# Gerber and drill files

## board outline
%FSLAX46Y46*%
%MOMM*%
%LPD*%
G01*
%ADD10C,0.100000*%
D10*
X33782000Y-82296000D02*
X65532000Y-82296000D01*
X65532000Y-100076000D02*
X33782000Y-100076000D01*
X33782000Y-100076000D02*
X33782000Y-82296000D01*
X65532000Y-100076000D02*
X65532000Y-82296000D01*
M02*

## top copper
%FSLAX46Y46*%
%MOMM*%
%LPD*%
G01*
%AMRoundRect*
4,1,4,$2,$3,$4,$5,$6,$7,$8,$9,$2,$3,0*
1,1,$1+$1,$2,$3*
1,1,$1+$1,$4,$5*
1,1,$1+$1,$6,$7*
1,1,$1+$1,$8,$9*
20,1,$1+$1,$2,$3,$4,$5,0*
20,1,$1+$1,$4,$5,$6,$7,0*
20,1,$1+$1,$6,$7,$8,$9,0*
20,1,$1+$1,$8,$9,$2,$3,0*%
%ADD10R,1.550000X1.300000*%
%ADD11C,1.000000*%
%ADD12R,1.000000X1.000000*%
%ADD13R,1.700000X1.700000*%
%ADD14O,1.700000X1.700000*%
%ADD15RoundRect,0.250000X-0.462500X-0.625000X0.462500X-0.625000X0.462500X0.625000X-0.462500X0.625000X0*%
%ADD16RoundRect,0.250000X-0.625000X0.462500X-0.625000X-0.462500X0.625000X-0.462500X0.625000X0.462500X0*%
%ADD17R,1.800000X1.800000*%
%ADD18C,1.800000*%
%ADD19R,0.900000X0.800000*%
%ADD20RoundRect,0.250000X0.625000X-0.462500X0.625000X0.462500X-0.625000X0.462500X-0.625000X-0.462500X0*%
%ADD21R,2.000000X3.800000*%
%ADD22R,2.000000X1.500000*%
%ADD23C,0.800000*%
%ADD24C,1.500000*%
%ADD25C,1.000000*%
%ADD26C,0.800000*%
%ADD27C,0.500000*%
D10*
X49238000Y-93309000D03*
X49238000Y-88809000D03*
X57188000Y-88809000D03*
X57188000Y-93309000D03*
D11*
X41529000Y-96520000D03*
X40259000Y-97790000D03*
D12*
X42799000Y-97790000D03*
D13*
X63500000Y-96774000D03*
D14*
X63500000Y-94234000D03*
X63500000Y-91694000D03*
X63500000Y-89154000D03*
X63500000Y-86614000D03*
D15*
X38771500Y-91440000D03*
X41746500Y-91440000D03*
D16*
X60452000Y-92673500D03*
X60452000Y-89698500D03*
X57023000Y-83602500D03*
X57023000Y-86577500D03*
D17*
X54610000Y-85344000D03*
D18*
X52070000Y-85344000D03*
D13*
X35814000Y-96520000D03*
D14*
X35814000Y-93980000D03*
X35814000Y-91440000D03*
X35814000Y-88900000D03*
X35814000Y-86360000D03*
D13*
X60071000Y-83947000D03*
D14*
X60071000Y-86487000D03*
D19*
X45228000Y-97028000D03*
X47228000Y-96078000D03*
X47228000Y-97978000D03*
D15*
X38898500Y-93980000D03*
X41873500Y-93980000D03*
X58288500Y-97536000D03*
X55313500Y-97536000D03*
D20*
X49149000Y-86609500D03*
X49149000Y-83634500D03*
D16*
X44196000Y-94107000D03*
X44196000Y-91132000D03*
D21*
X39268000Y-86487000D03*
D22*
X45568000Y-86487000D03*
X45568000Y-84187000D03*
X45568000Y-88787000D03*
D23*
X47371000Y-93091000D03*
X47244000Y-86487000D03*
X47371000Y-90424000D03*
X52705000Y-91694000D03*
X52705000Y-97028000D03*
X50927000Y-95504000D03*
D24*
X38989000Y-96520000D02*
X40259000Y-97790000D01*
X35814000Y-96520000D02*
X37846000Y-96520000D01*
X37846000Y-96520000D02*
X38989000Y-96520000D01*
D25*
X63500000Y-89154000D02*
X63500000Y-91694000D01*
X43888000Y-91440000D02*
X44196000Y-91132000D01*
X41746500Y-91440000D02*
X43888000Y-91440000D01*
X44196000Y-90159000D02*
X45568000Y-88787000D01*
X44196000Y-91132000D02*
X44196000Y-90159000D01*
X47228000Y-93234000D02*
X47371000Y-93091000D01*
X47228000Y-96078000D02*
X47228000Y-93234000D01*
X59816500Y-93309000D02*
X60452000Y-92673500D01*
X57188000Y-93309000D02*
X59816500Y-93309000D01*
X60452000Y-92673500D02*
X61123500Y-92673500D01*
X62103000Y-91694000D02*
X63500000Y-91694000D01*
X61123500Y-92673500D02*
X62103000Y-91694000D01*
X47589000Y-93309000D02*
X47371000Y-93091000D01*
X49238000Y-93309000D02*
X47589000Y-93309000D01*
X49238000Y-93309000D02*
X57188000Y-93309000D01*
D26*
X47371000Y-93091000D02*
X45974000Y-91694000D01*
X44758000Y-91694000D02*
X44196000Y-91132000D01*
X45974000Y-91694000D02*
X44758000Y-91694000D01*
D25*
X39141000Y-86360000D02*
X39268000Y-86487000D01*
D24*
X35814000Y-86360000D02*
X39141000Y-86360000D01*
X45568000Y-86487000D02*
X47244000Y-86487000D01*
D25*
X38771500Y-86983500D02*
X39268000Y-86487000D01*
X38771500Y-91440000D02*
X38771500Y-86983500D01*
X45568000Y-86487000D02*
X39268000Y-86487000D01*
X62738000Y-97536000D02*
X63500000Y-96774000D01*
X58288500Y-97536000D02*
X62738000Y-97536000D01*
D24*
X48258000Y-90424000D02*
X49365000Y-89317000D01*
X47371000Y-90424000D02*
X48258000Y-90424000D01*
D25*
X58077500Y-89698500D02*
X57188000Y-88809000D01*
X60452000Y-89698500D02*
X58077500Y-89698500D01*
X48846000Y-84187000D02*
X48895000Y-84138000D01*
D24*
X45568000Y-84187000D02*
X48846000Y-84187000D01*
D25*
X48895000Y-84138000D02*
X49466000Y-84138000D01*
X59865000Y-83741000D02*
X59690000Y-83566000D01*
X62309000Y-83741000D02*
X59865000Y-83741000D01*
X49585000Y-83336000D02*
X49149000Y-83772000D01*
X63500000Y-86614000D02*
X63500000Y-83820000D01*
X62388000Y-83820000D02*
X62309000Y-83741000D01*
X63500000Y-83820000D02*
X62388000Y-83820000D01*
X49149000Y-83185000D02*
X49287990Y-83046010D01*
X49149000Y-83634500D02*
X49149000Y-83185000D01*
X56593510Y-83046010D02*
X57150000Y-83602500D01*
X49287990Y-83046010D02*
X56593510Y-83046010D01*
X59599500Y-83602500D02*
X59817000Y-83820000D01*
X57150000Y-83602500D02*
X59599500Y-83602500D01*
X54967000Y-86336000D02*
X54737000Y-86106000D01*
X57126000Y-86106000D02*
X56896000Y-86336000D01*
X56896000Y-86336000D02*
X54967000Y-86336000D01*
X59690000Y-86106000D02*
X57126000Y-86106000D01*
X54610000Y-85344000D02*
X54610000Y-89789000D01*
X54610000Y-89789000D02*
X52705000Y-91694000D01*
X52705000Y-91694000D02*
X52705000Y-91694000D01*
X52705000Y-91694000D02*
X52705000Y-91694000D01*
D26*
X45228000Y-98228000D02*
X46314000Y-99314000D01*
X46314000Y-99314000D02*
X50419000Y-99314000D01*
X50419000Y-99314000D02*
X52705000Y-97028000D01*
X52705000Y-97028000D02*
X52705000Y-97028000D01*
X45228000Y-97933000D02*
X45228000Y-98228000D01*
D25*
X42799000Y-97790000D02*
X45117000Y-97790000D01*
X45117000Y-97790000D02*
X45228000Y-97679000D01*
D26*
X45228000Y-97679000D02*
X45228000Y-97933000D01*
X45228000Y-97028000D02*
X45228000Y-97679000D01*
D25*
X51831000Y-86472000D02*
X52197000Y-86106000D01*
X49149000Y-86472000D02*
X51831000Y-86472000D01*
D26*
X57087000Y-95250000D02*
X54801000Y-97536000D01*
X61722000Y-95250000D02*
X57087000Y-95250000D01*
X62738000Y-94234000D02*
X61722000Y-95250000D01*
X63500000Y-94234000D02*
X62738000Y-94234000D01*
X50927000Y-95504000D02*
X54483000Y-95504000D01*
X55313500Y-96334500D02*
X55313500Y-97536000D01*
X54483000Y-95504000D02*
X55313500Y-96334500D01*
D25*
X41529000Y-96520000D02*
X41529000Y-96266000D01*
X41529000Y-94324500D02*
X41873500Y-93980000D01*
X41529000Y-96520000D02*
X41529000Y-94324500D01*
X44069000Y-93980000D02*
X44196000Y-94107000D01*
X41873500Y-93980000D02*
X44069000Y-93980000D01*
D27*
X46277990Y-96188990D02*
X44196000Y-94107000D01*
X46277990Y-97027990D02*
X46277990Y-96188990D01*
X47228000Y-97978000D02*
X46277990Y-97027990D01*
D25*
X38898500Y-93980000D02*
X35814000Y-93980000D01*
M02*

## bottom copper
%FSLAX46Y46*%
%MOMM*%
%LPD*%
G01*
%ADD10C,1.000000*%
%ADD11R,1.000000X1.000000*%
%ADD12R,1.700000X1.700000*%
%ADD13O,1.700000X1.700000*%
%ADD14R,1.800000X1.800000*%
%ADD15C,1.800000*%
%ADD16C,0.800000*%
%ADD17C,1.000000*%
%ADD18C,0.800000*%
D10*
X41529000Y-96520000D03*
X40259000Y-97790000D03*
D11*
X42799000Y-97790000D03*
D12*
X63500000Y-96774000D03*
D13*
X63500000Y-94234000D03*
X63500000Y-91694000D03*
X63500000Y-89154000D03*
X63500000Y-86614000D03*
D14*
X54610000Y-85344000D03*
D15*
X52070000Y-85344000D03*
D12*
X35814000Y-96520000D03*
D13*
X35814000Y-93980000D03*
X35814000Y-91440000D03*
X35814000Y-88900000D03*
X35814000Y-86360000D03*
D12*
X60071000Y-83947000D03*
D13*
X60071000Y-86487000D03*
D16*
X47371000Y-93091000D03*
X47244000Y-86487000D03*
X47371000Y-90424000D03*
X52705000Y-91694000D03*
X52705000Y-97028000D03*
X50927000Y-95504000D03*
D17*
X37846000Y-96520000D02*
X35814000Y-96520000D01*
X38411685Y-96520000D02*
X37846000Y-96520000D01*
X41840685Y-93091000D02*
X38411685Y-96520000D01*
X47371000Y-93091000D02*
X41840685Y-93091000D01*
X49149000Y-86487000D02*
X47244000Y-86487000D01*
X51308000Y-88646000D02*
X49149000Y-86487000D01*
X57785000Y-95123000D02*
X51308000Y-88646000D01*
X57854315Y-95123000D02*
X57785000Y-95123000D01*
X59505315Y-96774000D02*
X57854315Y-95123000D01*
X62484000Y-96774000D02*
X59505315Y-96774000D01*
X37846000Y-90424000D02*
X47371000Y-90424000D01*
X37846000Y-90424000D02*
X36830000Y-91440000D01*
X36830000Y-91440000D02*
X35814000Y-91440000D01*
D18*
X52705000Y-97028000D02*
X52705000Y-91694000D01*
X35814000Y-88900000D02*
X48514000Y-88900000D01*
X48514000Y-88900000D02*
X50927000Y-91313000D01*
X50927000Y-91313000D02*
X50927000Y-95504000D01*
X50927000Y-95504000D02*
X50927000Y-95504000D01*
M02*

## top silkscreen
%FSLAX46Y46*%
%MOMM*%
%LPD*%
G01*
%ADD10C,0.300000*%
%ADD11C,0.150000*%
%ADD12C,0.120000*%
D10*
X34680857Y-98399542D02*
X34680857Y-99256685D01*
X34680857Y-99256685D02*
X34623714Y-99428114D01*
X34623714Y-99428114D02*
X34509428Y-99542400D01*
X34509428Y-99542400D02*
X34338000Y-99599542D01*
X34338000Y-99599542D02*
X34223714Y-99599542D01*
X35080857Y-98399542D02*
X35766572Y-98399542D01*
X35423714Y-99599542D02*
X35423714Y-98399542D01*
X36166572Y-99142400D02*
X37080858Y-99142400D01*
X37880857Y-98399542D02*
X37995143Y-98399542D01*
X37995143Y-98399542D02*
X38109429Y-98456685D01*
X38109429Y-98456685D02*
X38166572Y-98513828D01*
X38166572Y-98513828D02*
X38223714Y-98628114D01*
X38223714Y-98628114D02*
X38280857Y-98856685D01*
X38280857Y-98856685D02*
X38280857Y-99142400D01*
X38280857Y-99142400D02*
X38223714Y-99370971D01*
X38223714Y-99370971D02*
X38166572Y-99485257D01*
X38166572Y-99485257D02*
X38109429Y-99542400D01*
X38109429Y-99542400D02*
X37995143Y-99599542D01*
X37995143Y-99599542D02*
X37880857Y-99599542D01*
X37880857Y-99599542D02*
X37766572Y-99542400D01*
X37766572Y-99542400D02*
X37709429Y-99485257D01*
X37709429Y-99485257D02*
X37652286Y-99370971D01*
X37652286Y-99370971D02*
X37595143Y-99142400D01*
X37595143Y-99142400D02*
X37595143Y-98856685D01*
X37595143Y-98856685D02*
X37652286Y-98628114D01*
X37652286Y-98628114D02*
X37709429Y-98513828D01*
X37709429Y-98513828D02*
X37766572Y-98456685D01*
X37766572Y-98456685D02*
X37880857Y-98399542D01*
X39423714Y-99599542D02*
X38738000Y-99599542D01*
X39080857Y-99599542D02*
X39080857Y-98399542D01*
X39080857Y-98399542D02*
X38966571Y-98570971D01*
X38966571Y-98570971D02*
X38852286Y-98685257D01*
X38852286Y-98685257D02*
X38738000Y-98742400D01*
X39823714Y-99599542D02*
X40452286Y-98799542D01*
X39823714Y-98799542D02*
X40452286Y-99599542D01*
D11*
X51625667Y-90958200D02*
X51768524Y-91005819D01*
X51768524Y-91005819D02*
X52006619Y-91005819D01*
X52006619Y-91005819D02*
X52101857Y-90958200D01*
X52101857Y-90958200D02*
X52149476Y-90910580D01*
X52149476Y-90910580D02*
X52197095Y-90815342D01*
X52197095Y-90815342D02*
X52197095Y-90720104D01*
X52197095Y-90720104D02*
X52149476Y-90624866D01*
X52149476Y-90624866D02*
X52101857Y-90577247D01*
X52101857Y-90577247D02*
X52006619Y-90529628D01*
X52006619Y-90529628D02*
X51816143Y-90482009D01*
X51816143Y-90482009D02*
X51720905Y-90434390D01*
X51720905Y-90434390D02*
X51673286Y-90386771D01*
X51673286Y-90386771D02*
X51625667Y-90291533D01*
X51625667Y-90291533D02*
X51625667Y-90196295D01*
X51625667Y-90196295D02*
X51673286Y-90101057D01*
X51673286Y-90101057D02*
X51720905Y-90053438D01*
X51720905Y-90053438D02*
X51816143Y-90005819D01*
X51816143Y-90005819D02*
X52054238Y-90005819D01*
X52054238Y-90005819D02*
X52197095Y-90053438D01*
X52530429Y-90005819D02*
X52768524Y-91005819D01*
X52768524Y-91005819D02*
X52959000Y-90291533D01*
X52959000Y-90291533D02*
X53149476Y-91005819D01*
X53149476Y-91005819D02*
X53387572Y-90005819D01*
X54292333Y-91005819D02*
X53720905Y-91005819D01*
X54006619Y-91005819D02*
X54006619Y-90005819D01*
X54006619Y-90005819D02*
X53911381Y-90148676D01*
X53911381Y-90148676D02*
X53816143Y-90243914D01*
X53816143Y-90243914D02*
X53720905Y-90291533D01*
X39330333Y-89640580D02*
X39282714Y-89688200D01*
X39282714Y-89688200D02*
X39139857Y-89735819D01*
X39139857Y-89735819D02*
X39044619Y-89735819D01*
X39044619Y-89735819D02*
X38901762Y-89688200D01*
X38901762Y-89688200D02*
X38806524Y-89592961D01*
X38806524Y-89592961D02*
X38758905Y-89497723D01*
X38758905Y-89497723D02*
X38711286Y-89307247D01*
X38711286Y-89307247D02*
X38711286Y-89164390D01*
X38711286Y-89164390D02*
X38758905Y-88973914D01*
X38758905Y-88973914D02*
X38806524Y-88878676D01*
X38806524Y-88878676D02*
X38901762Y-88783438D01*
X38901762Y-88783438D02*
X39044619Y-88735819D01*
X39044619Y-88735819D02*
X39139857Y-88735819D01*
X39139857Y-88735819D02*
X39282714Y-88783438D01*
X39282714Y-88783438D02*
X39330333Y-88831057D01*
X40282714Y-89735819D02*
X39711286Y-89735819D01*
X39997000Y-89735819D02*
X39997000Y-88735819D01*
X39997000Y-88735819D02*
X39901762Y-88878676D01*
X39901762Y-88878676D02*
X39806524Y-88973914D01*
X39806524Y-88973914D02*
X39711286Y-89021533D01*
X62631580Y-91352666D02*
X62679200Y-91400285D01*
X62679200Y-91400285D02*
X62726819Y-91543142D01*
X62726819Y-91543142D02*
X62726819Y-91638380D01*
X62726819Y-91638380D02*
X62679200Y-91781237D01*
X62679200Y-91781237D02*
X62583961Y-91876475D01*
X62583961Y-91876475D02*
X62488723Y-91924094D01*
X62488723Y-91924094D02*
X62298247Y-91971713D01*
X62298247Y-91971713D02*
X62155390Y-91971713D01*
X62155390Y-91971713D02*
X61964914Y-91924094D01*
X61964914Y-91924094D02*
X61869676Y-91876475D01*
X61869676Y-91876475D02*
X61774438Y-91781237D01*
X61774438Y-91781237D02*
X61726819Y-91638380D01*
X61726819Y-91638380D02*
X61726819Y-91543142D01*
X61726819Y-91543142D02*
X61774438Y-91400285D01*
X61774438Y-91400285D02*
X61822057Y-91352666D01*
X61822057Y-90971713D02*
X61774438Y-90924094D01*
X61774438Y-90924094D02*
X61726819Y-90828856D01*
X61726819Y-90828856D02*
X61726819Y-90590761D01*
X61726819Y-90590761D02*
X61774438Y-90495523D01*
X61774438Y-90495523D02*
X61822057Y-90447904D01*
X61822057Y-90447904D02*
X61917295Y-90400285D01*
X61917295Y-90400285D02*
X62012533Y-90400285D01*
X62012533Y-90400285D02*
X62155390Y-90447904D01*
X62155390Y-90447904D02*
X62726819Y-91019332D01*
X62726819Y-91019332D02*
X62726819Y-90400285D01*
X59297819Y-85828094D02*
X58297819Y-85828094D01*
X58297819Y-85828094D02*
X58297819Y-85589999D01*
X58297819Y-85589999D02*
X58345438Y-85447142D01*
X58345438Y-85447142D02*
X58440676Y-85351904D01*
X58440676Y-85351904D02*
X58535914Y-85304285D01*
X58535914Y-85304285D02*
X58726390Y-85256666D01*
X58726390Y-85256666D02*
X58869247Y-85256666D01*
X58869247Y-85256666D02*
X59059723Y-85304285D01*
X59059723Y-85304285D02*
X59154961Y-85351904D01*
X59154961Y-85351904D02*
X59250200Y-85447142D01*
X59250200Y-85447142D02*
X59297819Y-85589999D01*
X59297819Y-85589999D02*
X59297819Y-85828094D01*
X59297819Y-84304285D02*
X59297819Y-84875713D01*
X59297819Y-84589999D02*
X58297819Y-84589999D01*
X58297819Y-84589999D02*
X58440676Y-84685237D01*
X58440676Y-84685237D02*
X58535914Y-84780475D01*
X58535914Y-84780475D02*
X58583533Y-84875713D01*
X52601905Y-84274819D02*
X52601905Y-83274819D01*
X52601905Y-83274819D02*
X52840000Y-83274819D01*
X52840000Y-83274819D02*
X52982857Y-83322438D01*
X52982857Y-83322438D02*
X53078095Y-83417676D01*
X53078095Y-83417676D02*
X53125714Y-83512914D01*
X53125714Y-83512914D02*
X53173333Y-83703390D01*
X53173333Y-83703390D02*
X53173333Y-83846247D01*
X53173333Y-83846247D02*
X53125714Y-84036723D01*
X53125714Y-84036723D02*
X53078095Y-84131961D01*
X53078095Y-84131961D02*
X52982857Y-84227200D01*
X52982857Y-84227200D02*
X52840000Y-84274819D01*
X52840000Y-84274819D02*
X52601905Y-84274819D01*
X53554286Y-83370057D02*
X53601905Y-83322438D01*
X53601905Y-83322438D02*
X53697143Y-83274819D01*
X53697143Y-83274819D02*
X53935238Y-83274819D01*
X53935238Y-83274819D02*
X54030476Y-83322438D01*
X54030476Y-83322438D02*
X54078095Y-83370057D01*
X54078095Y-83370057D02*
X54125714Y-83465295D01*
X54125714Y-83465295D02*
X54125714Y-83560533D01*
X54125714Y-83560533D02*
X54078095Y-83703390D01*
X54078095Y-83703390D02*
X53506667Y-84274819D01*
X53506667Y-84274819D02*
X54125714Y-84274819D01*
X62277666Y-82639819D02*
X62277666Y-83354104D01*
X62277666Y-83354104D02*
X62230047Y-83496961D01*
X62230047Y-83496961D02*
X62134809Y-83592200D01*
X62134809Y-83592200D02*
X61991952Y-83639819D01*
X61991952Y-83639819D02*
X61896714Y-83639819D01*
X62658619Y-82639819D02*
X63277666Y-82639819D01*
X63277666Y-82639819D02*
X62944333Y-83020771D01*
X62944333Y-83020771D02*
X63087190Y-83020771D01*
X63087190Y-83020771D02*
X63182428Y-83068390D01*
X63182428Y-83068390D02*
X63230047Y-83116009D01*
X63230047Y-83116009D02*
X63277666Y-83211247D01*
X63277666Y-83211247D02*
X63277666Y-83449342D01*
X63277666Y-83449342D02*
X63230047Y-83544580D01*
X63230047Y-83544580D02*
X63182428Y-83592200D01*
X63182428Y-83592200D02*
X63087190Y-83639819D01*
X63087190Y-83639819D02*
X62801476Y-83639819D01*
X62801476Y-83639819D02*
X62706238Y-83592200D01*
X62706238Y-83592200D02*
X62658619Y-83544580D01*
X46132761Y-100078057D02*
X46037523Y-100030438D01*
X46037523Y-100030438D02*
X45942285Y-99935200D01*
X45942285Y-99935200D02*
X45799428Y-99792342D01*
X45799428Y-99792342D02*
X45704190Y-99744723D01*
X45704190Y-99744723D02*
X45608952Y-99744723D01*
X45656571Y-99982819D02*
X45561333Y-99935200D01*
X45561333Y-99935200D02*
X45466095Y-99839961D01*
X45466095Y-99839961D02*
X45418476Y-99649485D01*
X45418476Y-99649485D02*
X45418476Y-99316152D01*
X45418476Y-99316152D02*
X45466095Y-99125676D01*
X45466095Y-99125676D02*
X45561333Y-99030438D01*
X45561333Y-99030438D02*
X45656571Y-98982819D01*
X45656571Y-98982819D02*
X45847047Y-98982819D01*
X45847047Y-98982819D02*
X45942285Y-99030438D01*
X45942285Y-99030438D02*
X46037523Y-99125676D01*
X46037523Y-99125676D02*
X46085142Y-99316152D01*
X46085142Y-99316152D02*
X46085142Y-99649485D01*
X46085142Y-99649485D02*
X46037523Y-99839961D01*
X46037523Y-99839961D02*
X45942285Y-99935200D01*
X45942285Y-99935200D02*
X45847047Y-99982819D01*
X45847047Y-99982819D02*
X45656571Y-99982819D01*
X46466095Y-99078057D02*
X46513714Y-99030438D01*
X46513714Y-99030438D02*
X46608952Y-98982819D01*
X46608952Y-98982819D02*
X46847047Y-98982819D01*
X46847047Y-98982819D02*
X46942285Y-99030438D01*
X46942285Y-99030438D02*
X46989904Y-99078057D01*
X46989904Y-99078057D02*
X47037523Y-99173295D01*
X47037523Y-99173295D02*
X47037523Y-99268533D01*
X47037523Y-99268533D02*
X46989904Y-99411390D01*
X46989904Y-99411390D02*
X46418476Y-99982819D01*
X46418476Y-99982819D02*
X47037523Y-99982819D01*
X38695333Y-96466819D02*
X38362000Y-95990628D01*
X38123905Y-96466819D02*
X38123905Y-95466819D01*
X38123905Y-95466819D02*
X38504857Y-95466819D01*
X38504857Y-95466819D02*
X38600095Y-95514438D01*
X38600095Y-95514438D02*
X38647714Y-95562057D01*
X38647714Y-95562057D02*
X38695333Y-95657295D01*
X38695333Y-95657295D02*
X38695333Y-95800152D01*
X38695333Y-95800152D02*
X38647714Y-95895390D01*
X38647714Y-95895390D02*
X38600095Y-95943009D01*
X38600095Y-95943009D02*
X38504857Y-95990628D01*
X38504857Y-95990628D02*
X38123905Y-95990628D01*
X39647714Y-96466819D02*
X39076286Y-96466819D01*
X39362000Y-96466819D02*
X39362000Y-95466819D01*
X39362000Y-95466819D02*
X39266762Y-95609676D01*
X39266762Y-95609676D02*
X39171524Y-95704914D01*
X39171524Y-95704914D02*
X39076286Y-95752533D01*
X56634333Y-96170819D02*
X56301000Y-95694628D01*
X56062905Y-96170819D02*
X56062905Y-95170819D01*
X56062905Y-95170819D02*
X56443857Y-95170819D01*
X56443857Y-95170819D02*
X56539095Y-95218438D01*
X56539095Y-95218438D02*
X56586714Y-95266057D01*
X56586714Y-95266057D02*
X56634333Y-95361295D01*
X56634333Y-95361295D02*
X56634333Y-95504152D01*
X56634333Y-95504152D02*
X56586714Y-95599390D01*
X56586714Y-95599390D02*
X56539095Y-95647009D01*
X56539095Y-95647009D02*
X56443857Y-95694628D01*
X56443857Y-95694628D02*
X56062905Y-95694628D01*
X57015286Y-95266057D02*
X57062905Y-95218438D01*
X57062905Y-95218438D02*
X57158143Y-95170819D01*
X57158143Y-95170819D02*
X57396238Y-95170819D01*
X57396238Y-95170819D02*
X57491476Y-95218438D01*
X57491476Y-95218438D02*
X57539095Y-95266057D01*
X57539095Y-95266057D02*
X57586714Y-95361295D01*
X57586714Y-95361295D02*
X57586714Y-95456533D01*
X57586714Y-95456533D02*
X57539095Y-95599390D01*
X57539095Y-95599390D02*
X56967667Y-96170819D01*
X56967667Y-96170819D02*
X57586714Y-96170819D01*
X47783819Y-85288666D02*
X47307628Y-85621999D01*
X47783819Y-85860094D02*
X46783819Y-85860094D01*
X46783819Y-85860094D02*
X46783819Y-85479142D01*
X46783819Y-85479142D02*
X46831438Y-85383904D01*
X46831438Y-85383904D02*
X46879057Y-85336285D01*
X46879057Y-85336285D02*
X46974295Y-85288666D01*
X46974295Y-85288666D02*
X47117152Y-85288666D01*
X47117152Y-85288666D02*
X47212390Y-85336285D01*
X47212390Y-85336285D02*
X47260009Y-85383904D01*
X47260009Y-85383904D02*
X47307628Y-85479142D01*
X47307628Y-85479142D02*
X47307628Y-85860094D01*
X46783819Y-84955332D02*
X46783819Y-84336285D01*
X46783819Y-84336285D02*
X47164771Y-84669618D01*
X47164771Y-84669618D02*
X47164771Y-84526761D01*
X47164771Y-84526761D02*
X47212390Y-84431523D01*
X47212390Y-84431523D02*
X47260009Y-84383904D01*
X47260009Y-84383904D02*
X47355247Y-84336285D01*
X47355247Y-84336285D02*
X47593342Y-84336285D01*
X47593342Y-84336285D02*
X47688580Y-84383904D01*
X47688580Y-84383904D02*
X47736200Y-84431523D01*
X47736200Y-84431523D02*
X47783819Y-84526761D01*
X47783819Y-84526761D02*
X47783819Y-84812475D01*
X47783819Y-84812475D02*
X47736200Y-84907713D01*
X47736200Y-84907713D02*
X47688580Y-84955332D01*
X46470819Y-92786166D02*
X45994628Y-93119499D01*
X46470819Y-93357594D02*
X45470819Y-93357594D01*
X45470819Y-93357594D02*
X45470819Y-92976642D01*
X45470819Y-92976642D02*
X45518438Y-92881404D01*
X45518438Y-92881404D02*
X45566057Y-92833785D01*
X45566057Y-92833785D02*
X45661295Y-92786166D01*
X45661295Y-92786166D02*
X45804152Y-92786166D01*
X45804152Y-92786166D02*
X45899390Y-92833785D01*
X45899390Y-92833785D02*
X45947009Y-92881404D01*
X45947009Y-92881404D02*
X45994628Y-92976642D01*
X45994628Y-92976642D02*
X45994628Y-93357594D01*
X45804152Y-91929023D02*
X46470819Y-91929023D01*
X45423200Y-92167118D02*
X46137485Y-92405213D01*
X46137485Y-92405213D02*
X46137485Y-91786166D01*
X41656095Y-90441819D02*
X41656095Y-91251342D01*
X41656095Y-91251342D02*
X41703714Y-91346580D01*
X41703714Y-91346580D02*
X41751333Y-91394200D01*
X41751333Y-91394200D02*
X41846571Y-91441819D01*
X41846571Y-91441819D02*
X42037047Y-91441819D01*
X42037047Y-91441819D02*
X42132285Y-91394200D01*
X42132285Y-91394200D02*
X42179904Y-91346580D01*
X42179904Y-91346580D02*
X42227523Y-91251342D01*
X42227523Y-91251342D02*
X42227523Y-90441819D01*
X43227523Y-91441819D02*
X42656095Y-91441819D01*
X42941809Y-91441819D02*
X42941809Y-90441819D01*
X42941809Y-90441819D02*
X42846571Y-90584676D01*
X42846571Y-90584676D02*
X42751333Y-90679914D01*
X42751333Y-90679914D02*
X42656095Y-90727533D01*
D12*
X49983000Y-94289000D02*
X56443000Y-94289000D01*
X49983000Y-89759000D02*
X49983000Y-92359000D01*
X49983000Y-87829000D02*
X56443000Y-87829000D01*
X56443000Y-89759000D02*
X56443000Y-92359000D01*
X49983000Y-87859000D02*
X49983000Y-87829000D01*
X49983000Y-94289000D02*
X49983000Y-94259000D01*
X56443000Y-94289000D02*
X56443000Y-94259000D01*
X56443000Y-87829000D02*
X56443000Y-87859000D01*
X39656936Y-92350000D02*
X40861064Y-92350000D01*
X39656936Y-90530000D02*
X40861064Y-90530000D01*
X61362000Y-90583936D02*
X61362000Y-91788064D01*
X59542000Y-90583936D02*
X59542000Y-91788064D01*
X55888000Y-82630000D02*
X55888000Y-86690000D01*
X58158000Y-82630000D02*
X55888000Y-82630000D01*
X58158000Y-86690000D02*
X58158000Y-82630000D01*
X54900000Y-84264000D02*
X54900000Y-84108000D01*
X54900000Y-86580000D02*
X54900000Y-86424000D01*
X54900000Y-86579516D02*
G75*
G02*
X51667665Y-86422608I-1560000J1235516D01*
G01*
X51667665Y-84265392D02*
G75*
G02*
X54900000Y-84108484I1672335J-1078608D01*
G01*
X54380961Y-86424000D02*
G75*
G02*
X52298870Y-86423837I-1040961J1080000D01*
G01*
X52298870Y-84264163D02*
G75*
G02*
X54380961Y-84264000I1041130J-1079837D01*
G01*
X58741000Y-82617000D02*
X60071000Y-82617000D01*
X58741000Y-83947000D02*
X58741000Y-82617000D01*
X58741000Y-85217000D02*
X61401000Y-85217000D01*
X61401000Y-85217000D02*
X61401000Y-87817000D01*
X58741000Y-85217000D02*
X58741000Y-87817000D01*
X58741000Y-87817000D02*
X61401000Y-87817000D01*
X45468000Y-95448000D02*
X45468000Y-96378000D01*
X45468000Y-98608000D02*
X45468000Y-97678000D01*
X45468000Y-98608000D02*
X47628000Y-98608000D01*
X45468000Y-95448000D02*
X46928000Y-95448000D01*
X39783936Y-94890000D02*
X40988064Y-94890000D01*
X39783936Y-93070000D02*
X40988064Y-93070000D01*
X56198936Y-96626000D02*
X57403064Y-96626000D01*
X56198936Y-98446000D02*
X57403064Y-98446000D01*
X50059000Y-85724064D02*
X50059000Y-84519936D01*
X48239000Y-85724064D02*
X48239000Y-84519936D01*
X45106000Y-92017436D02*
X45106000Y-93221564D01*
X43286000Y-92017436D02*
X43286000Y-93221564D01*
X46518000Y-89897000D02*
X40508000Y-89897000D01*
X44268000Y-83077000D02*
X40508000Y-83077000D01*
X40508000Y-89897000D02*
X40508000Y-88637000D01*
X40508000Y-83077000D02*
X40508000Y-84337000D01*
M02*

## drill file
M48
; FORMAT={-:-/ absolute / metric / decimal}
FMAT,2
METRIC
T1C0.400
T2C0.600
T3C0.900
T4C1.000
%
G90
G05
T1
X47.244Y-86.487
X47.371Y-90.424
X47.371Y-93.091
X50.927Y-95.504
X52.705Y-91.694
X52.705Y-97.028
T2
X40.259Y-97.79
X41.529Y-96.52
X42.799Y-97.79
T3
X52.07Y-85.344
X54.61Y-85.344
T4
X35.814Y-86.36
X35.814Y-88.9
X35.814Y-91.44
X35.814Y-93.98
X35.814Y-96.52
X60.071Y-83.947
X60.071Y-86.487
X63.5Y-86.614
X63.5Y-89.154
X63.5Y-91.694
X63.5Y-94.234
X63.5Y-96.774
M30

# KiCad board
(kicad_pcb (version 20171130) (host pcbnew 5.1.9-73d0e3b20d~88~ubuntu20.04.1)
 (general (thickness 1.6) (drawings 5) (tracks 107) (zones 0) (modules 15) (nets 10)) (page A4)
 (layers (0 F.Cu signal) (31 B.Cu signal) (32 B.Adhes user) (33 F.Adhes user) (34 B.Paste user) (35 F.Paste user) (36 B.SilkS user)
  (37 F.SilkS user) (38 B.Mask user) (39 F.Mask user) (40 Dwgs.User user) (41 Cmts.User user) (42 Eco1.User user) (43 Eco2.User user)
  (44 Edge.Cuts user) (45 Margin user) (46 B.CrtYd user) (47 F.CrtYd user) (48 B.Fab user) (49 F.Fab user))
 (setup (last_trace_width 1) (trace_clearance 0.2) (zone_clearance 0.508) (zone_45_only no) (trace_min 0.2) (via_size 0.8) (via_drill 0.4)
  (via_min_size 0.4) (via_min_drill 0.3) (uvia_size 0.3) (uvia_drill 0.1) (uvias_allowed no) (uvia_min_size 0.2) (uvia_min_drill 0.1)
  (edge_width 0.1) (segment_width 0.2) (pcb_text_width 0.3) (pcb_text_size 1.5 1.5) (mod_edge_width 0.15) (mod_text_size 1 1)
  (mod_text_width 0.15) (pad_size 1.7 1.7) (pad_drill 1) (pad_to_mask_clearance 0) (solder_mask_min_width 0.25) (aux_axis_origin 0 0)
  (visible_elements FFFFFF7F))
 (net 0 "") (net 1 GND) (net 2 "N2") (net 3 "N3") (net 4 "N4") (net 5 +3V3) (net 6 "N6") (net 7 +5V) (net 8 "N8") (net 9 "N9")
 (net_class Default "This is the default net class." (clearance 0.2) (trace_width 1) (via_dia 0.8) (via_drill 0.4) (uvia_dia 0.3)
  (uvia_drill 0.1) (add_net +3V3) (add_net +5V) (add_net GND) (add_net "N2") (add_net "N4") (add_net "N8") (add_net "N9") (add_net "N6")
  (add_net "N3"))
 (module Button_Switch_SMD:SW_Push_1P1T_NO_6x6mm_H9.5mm (layer F.Cu) (at 53.213 91.059)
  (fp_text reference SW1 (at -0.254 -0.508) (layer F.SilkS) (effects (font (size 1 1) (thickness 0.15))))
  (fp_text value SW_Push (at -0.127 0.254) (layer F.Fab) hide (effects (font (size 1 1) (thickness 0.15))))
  (fp_line (start -3.23 3.23) (end 3.23 3.23) (layer F.SilkS) (width 0.12))
  (fp_line (start -3.23 -1.3) (end -3.23 1.3) (layer F.SilkS) (width 0.12))
  (fp_line (start -3.23 -3.23) (end 3.23 -3.23) (layer F.SilkS) (width 0.12))
  (fp_line (start 3.23 -1.3) (end 3.23 1.3) (layer F.SilkS) (width 0.12))
  (fp_line (start -3.23 -3.2) (end -3.23 -3.23) (layer F.SilkS) (width 0.12))
  (fp_line (start -3.23 3.23) (end -3.23 3.2) (layer F.SilkS) (width 0.12))
  (fp_line (start 3.23 3.23) (end 3.23 3.2) (layer F.SilkS) (width 0.12))
  (fp_line (start 3.23 -3.23) (end 3.23 -3.2) (layer F.SilkS) (width 0.12))
  (pad 2 smd rect (at -3.975 2.25) (size 1.55 1.3) (layers F.Cu F.Paste F.Mask) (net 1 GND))
  (pad 1 smd rect (at -3.975 -2.25) (size 1.55 1.3) (layers F.Cu F.Paste F.Mask) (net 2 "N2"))
  (pad 1 smd rect (at 3.975 -2.25) (size 1.55 1.3) (layers F.Cu F.Paste F.Mask) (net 2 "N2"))
  (pad 2 smd rect (at 3.975 2.25) (size 1.55 1.3) (layers F.Cu F.Paste F.Mask) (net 1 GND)))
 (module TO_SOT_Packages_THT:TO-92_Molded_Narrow (layer B.Cu) (at 42.799 97.79 180)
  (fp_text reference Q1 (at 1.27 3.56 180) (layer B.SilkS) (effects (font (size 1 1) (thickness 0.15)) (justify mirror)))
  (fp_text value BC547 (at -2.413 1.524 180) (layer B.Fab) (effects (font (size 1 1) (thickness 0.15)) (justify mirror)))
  (pad 2 thru_hole circle (at 1.27 1.27 90) (size 1 1) (drill 0.6) (layers *.Cu *.Mask) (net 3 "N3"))
  (pad 3 thru_hole circle (at 2.54 0 90) (size 1 1) (drill 0.6) (layers *.Cu *.Mask) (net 1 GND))
  (pad 1 thru_hole rect (at 0 0 90) (size 1 1) (drill 0.6) (layers *.Cu *.Mask) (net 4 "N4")))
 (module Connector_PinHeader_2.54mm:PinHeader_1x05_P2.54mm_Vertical (layer B.Cu) (at 63.5 96.774)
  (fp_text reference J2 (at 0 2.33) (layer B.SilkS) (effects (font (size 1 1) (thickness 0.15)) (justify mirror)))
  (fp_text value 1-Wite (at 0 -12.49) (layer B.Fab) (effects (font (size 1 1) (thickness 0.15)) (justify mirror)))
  (pad 1 thru_hole rect (at 0 0) (size 1.7 1.7) (drill 1) (layers *.Cu *.Mask) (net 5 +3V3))
  (pad 2 thru_hole oval (at 0 -2.54) (size 1.7 1.7) (drill 1) (layers *.Cu *.Mask) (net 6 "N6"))
  (pad 3 thru_hole oval (at 0 -5.08) (size 1.7 1.7) (drill 1) (layers *.Cu *.Mask) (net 1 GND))
  (pad 4 thru_hole oval (at 0 -7.62) (size 1.7 1.7) (drill 1) (layers *.Cu *.Mask) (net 1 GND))
  (pad 5 thru_hole oval (at 0 -10.16) (size 1.7 1.7) (drill 1) (layers *.Cu *.Mask) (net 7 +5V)))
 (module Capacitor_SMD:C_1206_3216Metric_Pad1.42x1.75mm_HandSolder (layer F.Cu) (at 40.259 91.44)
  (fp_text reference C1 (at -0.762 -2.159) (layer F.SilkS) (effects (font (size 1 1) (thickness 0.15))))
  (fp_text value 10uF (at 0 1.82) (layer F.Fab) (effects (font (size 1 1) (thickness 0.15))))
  (fp_line (start -0.602064 0.91) (end 0.602064 0.91) (layer F.SilkS) (width 0.12))
  (fp_line (start -0.602064 -0.91) (end 0.602064 -0.91) (layer F.SilkS) (width 0.12))
  (pad 1 smd roundrect (at -1.4875 0) (size 1.425 1.75) (layers F.Cu F.Paste F.Mask) (roundrect_rratio 0.1754385964912281) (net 5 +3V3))
  (pad 2 smd roundrect (at 1.4875 0) (size 1.425 1.75) (layers F.Cu F.Paste F.Mask) (roundrect_rratio 0.1754385964912281) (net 1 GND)))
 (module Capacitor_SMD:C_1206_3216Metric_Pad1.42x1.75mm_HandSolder (layer F.Cu) (at 60.452 91.186 270)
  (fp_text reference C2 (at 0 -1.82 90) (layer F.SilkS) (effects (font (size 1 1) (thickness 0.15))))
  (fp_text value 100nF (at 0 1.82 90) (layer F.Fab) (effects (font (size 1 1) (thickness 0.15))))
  (fp_line (start -0.602064 -0.91) (end 0.602064 -0.91) (layer F.SilkS) (width 0.12))
  (fp_line (start -0.602064 0.91) (end 0.602064 0.91) (layer F.SilkS) (width 0.12))
  (pad 2 smd roundrect (at 1.4875 0 270) (size 1.425 1.75) (layers F.Cu F.Paste F.Mask) (roundrect_rratio 0.1754385964912281) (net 1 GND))
  (pad 1 smd roundrect (at -1.4875 0 270) (size 1.425 1.75) (layers F.Cu F.Paste F.Mask) (roundrect_rratio 0.1754385964912281) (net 2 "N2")))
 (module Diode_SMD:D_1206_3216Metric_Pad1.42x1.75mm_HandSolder (layer F.Cu) (at 57.023 85.09 270)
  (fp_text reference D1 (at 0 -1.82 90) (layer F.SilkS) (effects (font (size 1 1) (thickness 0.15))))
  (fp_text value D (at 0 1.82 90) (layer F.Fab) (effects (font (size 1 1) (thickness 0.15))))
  (fp_line (start -2.46 1.135) (end 1.6 1.135) (layer F.SilkS) (width 0.12))
  (fp_line (start -2.46 -1.135) (end -2.46 1.135) (layer F.SilkS) (width 0.12))
  (fp_line (start 1.6 -1.135) (end -2.46 -1.135) (layer F.SilkS) (width 0.12))
  (pad 1 smd roundrect (at -1.4875 0 270) (size 1.425 1.75) (layers F.Cu F.Paste F.Mask) (roundrect_rratio 0.1754385964912281) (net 7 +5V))
  (pad 2 smd roundrect (at 1.4875 0 270) (size 1.425 1.75) (layers F.Cu F.Paste F.Mask) (roundrect_rratio 0.1754385964912281) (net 4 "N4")))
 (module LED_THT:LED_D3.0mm (layer F.Cu) (at 54.61 85.344 180)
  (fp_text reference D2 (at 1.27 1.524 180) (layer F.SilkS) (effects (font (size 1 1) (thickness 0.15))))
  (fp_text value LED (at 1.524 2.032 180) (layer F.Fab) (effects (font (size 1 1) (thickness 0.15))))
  (fp_line (start -0.29 1.08) (end -0.29 1.236) (layer F.SilkS) (width 0.12))
  (fp_line (start -0.29 -1.236) (end -0.29 -1.08) (layer F.SilkS) (width 0.12))
  (fp_arc (start 1.27 0) (end -0.29 -1.235516) (angle 108.8) (layer F.SilkS) (width 0.12))
  (fp_arc (start 1.27 0) (end -0.29 1.235516) (angle -108.8) (layer F.SilkS) (width 0.12))
  (fp_arc (start 1.27 0) (end 0.229039 -1.08) (angle 87.9) (layer F.SilkS) (width 0.12))
  (fp_arc (start 1.27 0) (end 0.229039 1.08) (angle -87.9) (layer F.SilkS) (width 0.12))
  (pad 1 thru_hole rect (at 0 0 180) (size 1.8 1.8) (drill 0.9) (layers *.Cu *.Mask) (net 4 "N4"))
  (pad 2 thru_hole circle (at 2.54 0 180) (size 1.8 1.8) (drill 0.9) (layers *.Cu *.Mask) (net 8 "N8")))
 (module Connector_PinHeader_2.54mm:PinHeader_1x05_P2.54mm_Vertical (layer B.Cu) (at 35.814 96.52)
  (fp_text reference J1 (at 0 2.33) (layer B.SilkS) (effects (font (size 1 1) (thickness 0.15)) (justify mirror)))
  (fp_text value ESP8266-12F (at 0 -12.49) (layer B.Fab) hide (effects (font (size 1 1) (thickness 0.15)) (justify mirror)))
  (pad 1 thru_hole rect (at 0 0) (size 1.7 1.7) (drill 1) (layers *.Cu *.Mask) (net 1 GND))
  (pad 2 thru_hole oval (at 0 -2.54) (size 1.7 1.7) (drill 1) (layers *.Cu *.Mask) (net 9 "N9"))
  (pad 3 thru_hole oval (at 0 -5.08) (size 1.7 1.7) (drill 1) (layers *.Cu *.Mask) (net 2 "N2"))
  (pad 4 thru_hole oval (at 0 -7.62) (size 1.7 1.7) (drill 1) (layers *.Cu *.Mask) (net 6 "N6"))
  (pad 5 thru_hole oval (at 0 -10.16) (size 1.7 1.7) (drill 1) (layers *.Cu *.Mask) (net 5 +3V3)))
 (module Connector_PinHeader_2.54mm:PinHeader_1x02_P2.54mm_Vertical (layer F.Cu) (at 60.071 83.947)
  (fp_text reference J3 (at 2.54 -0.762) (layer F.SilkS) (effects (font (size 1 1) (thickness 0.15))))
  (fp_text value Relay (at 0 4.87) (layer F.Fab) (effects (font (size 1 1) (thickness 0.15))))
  (fp_line (start -1.33 -1.33) (end 0 -1.33) (layer F.SilkS) (width 0.12))
  (fp_line (start -1.33 0) (end -1.33 -1.33) (layer F.SilkS) (width 0.12))
  (fp_line (start -1.33 1.27) (end 1.33 1.27) (layer F.SilkS) (width 0.12))
  (fp_line (start 1.33 1.27) (end 1.33 3.87) (layer F.SilkS) (width 0.12))
  (fp_line (start -1.33 1.27) (end -1.33 3.87) (layer F.SilkS) (width 0.12))
  (fp_line (start -1.33 3.87) (end 1.33 3.87) (layer F.SilkS) (width 0.12))
  (pad 1 thru_hole rect (at 0 0) (size 1.7 1.7) (drill 1) (layers *.Cu *.Mask) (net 7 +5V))
  (pad 2 thru_hole oval (at 0 2.54) (size 1.7 1.7) (drill 1) (layers *.Cu *.Mask) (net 4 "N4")))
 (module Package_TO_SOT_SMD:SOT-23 (layer F.Cu) (at 46.228 97.028 180)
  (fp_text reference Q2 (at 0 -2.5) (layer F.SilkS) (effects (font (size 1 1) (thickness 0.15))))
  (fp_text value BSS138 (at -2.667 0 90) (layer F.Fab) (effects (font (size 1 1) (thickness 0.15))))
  (fp_line (start 0.76 1.58) (end 0.76 0.65) (layer F.SilkS) (width 0.12))
  (fp_line (start 0.76 -1.58) (end 0.76 -0.65) (layer F.SilkS) (width 0.12))
  (fp_line (start 0.76 -1.58) (end -1.4 -1.58) (layer F.SilkS) (width 0.12))
  (fp_line (start 0.76 1.58) (end -0.7 1.58) (layer F.SilkS) (width 0.12))
  (pad 3 smd rect (at 1 0 180) (size 0.9 0.8) (layers F.Cu F.Paste F.Mask) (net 4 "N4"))
  (pad 2 smd rect (at -1 0.95 180) (size 0.9 0.8) (layers F.Cu F.Paste F.Mask) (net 1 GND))
  (pad 1 smd rect (at -1 -0.95 180) (size 0.9 0.8) (layers F.Cu F.Paste F.Mask) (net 3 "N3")))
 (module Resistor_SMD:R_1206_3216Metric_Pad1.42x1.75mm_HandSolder (layer F.Cu) (at 40.386 93.98)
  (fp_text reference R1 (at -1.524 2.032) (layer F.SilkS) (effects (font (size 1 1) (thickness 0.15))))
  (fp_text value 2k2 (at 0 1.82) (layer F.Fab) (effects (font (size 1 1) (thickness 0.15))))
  (fp_line (start -0.602064 0.91) (end 0.602064 0.91) (layer F.SilkS) (width 0.12))
  (fp_line (start -0.602064 -0.91) (end 0.602064 -0.91) (layer F.SilkS) (width 0.12))
  (pad 1 smd roundrect (at -1.4875 0) (size 1.425 1.75) (layers F.Cu F.Paste F.Mask) (roundrect_rratio 0.1754385964912281) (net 9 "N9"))
  (pad 2 smd roundrect (at 1.4875 0) (size 1.425 1.75) (layers F.Cu F.Paste F.Mask) (roundrect_rratio 0.1754385964912281) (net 3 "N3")))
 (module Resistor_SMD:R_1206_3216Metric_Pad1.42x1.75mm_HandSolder (layer F.Cu) (at 56.801 97.536)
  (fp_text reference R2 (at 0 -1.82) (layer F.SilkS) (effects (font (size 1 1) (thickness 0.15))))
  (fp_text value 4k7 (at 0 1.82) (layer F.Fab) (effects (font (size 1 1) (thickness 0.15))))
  (fp_line (start -0.602064 -0.91) (end 0.602064 -0.91) (layer F.SilkS) (width 0.12))
  (fp_line (start -0.602064 0.91) (end 0.602064 0.91) (layer F.SilkS) (width 0.12))
  (pad 2 smd roundrect (at 1.4875 0) (size 1.425 1.75) (layers F.Cu F.Paste F.Mask) (roundrect_rratio 0.1754385964912281) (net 5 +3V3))
  (pad 1 smd roundrect (at -1.4875 0) (size 1.425 1.75) (layers F.Cu F.Paste F.Mask) (roundrect_rratio 0.1754385964912281) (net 6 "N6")))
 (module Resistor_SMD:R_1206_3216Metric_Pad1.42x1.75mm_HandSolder (layer F.Cu) (at 49.149 85.122 90)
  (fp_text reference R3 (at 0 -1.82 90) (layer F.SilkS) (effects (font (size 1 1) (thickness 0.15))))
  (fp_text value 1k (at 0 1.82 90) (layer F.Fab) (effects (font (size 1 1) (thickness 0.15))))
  (fp_line (start -0.602064 0.91) (end 0.602064 0.91) (layer F.SilkS) (width 0.12))
  (fp_line (start -0.602064 -0.91) (end 0.602064 -0.91) (layer F.SilkS) (width 0.12))
  (pad 1 smd roundrect (at -1.4875 0 90) (size 1.425 1.75) (layers F.Cu F.Paste F.Mask) (roundrect_rratio 0.1754385964912281) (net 8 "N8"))
  (pad 2 smd roundrect (at 1.4875 0 90) (size 1.425 1.75) (layers F.Cu F.Paste F.Mask) (roundrect_rratio 0.1754385964912281) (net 7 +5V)))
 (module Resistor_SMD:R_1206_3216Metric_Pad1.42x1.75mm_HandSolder (layer F.Cu) (at 44.196 92.6195 270)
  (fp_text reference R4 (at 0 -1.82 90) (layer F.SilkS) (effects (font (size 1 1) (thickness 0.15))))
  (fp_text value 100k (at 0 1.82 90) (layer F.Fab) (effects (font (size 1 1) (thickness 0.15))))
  (fp_line (start -0.602064 -0.91) (end 0.602064 -0.91) (layer F.SilkS) (width 0.12))
  (fp_line (start -0.602064 0.91) (end 0.602064 0.91) (layer F.SilkS) (width 0.12))
  (pad 2 smd roundrect (at 1.4875 0 270) (size 1.425 1.75) (layers F.Cu F.Paste F.Mask) (roundrect_rratio 0.1754385964912281) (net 3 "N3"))
  (pad 1 smd roundrect (at -1.4875 0 270) (size 1.425 1.75) (layers F.Cu F.Paste F.Mask) (roundrect_rratio 0.1754385964912281) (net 1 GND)))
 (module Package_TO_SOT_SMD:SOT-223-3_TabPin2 (layer F.Cu) (at 42.418 86.487 180)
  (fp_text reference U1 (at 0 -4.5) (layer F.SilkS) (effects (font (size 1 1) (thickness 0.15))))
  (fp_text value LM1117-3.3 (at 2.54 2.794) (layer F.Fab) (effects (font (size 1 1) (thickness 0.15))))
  (fp_line (start -4.1 -3.41) (end 1.91 -3.41) (layer F.SilkS) (width 0.12))
  (fp_line (start -1.85 3.41) (end 1.91 3.41) (layer F.SilkS) (width 0.12))
  (fp_line (start 1.91 -3.41) (end 1.91 -2.15) (layer F.SilkS) (width 0.12))
  (fp_line (start 1.91 3.41) (end 1.91 2.15) (layer F.SilkS) (width 0.12))
  (pad 2 smd rect (at 3.15 0 180) (size 2 3.8) (layers F.Cu F.Paste F.Mask) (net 5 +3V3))
  (pad 2 smd rect (at -3.15 0 180) (size 2 1.5) (layers F.Cu F.Paste F.Mask) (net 5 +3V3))
  (pad 3 smd rect (at -3.15 2.3 180) (size 2 1.5) (layers F.Cu F.Paste F.Mask) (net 7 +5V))
  (pad 1 smd rect (at -3.15 -2.3 180) (size 2 1.5) (layers F.Cu F.Paste F.Mask) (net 1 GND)))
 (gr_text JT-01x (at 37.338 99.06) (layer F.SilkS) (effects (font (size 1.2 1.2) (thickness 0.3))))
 (gr_line (start 33.782 82.296) (end 65.532 82.296) (layer Edge.Cuts) (width 0.1))
 (gr_line (start 65.532 100.076) (end 33.782 100.076) (layer Edge.Cuts) (width 0.1))
 (gr_line (start 33.782 100.076) (end 33.782 82.296) (layer Edge.Cuts) (width 0.1))
 (gr_line (start 65.532 100.076) (end 65.532 82.296) (layer Edge.Cuts) (width 0.1))
 (segment (start 38.989 96.52) (end 40.259 97.79) (width 1.5) (layer F.Cu) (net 1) (status 20))
 (segment (start 35.814 96.52) (end 37.846 96.52) (width 1.5) (layer F.Cu) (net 1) (status 10))
 (segment (start 37.846 96.52) (end 38.989 96.52) (width 1.5) (layer F.Cu) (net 1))
 (via (at 47.371 93.091) (size 0.8) (drill 0.4) (layers F.Cu B.Cu) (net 1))
 (segment (start 37.846 96.52) (end 35.814 96.52) (width 1) (layer B.Cu) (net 1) (status 20))
 (segment (start 38.411685 96.52) (end 37.846 96.52) (width 1) (layer B.Cu) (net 1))
 (segment (start 41.840685 93.091) (end 38.411685 96.52) (width 1) (layer B.Cu) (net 1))
 (segment (start 47.371 93.091) (end 41.840685 93.091) (width 1) (layer B.Cu) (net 1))
 (segment (start 63.5 89.154) (end 63.5 91.694) (width 1) (layer F.Cu) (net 1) (status 30))
 (segment (start 43.888 91.44) (end 44.196 91.132) (width 1) (layer F.Cu) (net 1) (status 30))
 (segment (start 41.7465 91.44) (end 43.888 91.44) (width 1) (layer F.Cu) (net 1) (status 30))
 (segment (start 44.196 90.159) (end 45.568 88.787) (width 1) (layer F.Cu) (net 1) (status 20))
 (segment (start 44.196 91.132) (end 44.196 90.159) (width 1) (layer F.Cu) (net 1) (status 10))
 (segment (start 47.228 93.234) (end 47.371 93.091) (width 1) (layer F.Cu) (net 1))
 (segment (start 47.228 96.078) (end 47.228 93.234) (width 1) (layer F.Cu) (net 1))
 (segment (start 59.8165 93.309) (end 60.452 92.6735) (width 1) (layer F.Cu) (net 1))
 (segment (start 57.188 93.309) (end 59.8165 93.309) (width 1) (layer F.Cu) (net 1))
 (segment (start 60.452 92.6735) (end 61.1235 92.6735) (width 1) (layer F.Cu) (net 1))
 (segment (start 62.103 91.694) (end 63.5 91.694) (width 1) (layer F.Cu) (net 1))
 (segment (start 61.1235 92.6735) (end 62.103 91.694) (width 1) (layer F.Cu) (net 1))
 (segment (start 47.589 93.309) (end 47.371 93.091) (width 1) (layer F.Cu) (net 1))
 (segment (start 49.238 93.309) (end 47.589 93.309) (width 1) (layer F.Cu) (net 1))
 (segment (start 49.238 93.309) (end 57.188 93.309) (width 1) (layer F.Cu) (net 1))
 (segment (start 47.371 93.091) (end 45.974 91.694) (width 0.8) (layer F.Cu) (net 1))
 (segment (start 44.758 91.694) (end 44.196 91.132) (width 0.8) (layer F.Cu) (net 1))
 (segment (start 45.974 91.694) (end 44.758 91.694) (width 0.8) (layer F.Cu) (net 1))
 (segment (start 39.141 86.36) (end 39.268 86.487) (width 1) (layer F.Cu) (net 5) (status 30))
 (segment (start 35.814 86.36) (end 39.141 86.36) (width 1.5) (layer F.Cu) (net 5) (status 30))
 (segment (start 45.568 86.487) (end 47.244 86.487) (width 1.5) (layer F.Cu) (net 5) (status 10))
 (via (at 47.244 86.487) (size 0.8) (drill 0.4) (layers F.Cu B.Cu) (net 5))
 (segment (start 49.149 86.487) (end 47.244 86.487) (width 1) (layer B.Cu) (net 5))
 (segment (start 51.308 88.646) (end 49.149 86.487) (width 1) (layer B.Cu) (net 5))
 (segment (start 57.785 95.123) (end 51.308 88.646) (width 1) (layer B.Cu) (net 5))
 (segment (start 57.854315 95.123) (end 57.785 95.123) (width 1) (layer B.Cu) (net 5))
 (segment (start 59.505315 96.774) (end 57.854315 95.123) (width 1) (layer B.Cu) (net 5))
 (segment (start 62.484 96.774) (end 59.505315 96.774) (width 1) (layer B.Cu) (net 5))
 (segment (start 38.7715 86.9835) (end 39.268 86.487) (width 1) (layer F.Cu) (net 5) (status 30))
 (segment (start 38.7715 91.44) (end 38.7715 86.9835) (width 1) (layer F.Cu) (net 5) (status 30))
 (segment (start 45.568 86.487) (end 39.268 86.487) (width 1) (layer F.Cu) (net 5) (status 30))
 (segment (start 62.738 97.536) (end 63.5 96.774) (width 1) (layer F.Cu) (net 5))
 (segment (start 58.2885 97.536) (end 62.738 97.536) (width 1) (layer F.Cu) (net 5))
 (via (at 47.371 90.424) (size 0.8) (drill 0.4) (layers F.Cu B.Cu) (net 2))
 (segment (start 37.846 90.424) (end 47.371 90.424) (width 1) (layer B.Cu) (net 2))
 (segment (start 48.258 90.424) (end 49.365 89.317) (width 1.5) (layer F.Cu) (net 2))
 (segment (start 47.371 90.424) (end 48.258 90.424) (width 1.5) (layer F.Cu) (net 2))
 (segment (start 37.846 90.424) (end 36.83 91.44) (width 1) (layer B.Cu) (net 2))
 (segment (start 36.83 91.44) (end 35.814 91.44) (width 1) (layer B.Cu) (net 2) (status 20))
 (segment (start 58.0775 89.6985) (end 57.188 88.809) (width 1) (layer F.Cu) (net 2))
 (segment (start 60.452 89.6985) (end 58.0775 89.6985) (width 1) (layer F.Cu) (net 2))
 (segment (start 48.846 84.187) (end 48.895 84.138) (width 1) (layer F.Cu) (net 7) (status 30))
 (segment (start 45.568 84.187) (end 48.846 84.187) (width 1.5) (layer F.Cu) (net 7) (status 30))
 (segment (start 48.895 84.138) (end 49.466 84.138) (width 1) (layer F.Cu) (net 7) (status 30))
 (segment (start 59.865 83.741) (end 59.69 83.566) (width 1) (layer F.Cu) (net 7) (status 30))
 (segment (start 62.309 83.741) (end 59.865 83.741) (width 1) (layer F.Cu) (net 7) (status 20))
 (segment (start 49.585 83.336) (end 49.149 83.772) (width 1) (layer F.Cu) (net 7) (status 30))
 (segment (start 63.5 86.614) (end 63.5 83.82) (width 1) (layer F.Cu) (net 7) (status 10))
 (segment (start 62.388 83.82) (end 62.309 83.741) (width 1) (layer F.Cu) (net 7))
 (segment (start 63.5 83.82) (end 62.388 83.82) (width 1) (layer F.Cu) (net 7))
 (segment (start 49.149 83.185) (end 49.28799 83.04601) (width 1) (layer F.Cu) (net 7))
 (segment (start 49.149 83.6345) (end 49.149 83.185) (width 1) (layer F.Cu) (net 7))
 (segment (start 56.59351 83.04601) (end 57.15 83.6025) (width 1) (layer F.Cu) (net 7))
 (segment (start 49.28799 83.04601) (end 56.59351 83.04601) (width 1) (layer F.Cu) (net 7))
 (segment (start 59.5995 83.6025) (end 59.817 83.82) (width 1) (layer F.Cu) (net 7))
 (segment (start 57.15 83.6025) (end 59.5995 83.6025) (width 1) (layer F.Cu) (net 7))
 (segment (start 54.967 86.336) (end 54.737 86.106) (width 1) (layer F.Cu) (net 4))
 (segment (start 57.126 86.106) (end 56.896 86.336) (width 1) (layer F.Cu) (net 4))
 (segment (start 56.896 86.336) (end 54.967 86.336) (width 1) (layer F.Cu) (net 4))
 (segment (start 59.69 86.106) (end 57.126 86.106) (width 1) (layer F.Cu) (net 4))
 (segment (start 54.61 85.344) (end 54.61 89.789) (width 1) (layer F.Cu) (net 4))
 (segment (start 54.61 89.789) (end 52.705 91.694) (width 1) (layer F.Cu) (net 4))
 (segment (start 52.705 91.694) (end 52.705 91.694) (width 1) (layer F.Cu) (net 4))
 (segment (start 52.705 91.694) (end 52.705 91.694) (width 1) (layer F.Cu) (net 4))
 (via (at 52.705 91.694) (size 0.8) (drill 0.4) (layers F.Cu B.Cu) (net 4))
 (segment (start 45.228 98.228) (end 46.314 99.314) (width 0.8) (layer F.Cu) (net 4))
 (segment (start 46.314 99.314) (end 50.419 99.314) (width 0.8) (layer F.Cu) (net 4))
 (segment (start 50.419 99.314) (end 52.705 97.028) (width 0.8) (layer F.Cu) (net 4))
 (segment (start 52.705 97.028) (end 52.705 97.028) (width 0.8) (layer F.Cu) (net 4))
 (via (at 52.705 97.028) (size 0.8) (drill 0.4) (layers F.Cu B.Cu) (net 4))
 (segment (start 52.705 97.028) (end 52.705 91.694) (width 0.8) (layer B.Cu) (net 4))
 (segment (start 45.228 97.933) (end 45.228 98.228) (width 0.8) (layer F.Cu) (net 4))
 (segment (start 42.799 97.79) (end 45.117 97.79) (width 1) (layer F.Cu) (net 4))
 (segment (start 45.117 97.79) (end 45.228 97.679) (width 1) (layer F.Cu) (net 4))
 (segment (start 45.228 97.679) (end 45.228 97.933) (width 0.8) (layer F.Cu) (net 4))
 (segment (start 45.228 97.028) (end 45.228 97.679) (width 0.8) (layer F.Cu) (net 4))
 (segment (start 51.831 86.472) (end 52.197 86.106) (width 1) (layer F.Cu) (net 8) (status 20))
 (segment (start 49.149 86.472) (end 51.831 86.472) (width 1) (layer F.Cu) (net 8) (status 10))
 (segment (start 57.087 95.25) (end 54.801 97.536) (width 0.8) (layer F.Cu) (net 6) (status 20))
 (segment (start 61.722 95.25) (end 57.087 95.25) (width 0.8) (layer F.Cu) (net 6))
 (segment (start 62.738 94.234) (end 61.722 95.25) (width 0.8) (layer F.Cu) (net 6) (status 10))
 (segment (start 63.5 94.234) (end 62.738 94.234) (width 0.8) (layer F.Cu) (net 6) (status 30))
 (segment (start 35.814 88.9) (end 48.514 88.9) (width 0.8) (layer B.Cu) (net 6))
 (segment (start 48.514 88.9) (end 50.927 91.313) (width 0.8) (layer B.Cu) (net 6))
 (segment (start 50.927 91.313) (end 50.927 95.504) (width 0.8) (layer B.Cu) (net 6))
 (segment (start 50.927 95.504) (end 50.927 95.504) (width 0.8) (layer B.Cu) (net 6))
 (via (at 50.927 95.504) (size 0.8) (drill 0.4) (layers F.Cu B.Cu) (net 6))
 (segment (start 50.927 95.504) (end 54.483 95.504) (width 0.8) (layer F.Cu) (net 6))
 (segment (start 55.3135 96.3345) (end 55.3135 97.536) (width 0.8) (layer F.Cu) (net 6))
 (segment (start 54.483 95.504) (end 55.3135 96.3345) (width 0.8) (layer F.Cu) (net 6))
 (segment (start 41.529 96.52) (end 41.529 96.266) (width 1) (layer F.Cu) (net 3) (status 30))
 (segment (start 41.529 94.3245) (end 41.8735 93.98) (width 1) (layer F.Cu) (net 3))
 (segment (start 41.529 96.52) (end 41.529 94.3245) (width 1) (layer F.Cu) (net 3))
 (segment (start 44.069 93.98) (end 44.196 94.107) (width 1) (layer F.Cu) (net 3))
 (segment (start 41.8735 93.98) (end 44.069 93.98) (width 1) (layer F.Cu) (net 3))
 (segment (start 46.27799 96.18899) (end 44.196 94.107) (width 0.5) (layer F.Cu) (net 3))
 (segment (start 46.27799 97.02799) (end 46.27799 96.18899) (width 0.5) (layer F.Cu) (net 3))
 (segment (start 47.228 97.978) (end 46.27799 97.02799) (width 0.5) (layer F.Cu) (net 3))
 (segment (start 38.8985 93.98) (end 35.814 93.98) (width 1) (layer F.Cu) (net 9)))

